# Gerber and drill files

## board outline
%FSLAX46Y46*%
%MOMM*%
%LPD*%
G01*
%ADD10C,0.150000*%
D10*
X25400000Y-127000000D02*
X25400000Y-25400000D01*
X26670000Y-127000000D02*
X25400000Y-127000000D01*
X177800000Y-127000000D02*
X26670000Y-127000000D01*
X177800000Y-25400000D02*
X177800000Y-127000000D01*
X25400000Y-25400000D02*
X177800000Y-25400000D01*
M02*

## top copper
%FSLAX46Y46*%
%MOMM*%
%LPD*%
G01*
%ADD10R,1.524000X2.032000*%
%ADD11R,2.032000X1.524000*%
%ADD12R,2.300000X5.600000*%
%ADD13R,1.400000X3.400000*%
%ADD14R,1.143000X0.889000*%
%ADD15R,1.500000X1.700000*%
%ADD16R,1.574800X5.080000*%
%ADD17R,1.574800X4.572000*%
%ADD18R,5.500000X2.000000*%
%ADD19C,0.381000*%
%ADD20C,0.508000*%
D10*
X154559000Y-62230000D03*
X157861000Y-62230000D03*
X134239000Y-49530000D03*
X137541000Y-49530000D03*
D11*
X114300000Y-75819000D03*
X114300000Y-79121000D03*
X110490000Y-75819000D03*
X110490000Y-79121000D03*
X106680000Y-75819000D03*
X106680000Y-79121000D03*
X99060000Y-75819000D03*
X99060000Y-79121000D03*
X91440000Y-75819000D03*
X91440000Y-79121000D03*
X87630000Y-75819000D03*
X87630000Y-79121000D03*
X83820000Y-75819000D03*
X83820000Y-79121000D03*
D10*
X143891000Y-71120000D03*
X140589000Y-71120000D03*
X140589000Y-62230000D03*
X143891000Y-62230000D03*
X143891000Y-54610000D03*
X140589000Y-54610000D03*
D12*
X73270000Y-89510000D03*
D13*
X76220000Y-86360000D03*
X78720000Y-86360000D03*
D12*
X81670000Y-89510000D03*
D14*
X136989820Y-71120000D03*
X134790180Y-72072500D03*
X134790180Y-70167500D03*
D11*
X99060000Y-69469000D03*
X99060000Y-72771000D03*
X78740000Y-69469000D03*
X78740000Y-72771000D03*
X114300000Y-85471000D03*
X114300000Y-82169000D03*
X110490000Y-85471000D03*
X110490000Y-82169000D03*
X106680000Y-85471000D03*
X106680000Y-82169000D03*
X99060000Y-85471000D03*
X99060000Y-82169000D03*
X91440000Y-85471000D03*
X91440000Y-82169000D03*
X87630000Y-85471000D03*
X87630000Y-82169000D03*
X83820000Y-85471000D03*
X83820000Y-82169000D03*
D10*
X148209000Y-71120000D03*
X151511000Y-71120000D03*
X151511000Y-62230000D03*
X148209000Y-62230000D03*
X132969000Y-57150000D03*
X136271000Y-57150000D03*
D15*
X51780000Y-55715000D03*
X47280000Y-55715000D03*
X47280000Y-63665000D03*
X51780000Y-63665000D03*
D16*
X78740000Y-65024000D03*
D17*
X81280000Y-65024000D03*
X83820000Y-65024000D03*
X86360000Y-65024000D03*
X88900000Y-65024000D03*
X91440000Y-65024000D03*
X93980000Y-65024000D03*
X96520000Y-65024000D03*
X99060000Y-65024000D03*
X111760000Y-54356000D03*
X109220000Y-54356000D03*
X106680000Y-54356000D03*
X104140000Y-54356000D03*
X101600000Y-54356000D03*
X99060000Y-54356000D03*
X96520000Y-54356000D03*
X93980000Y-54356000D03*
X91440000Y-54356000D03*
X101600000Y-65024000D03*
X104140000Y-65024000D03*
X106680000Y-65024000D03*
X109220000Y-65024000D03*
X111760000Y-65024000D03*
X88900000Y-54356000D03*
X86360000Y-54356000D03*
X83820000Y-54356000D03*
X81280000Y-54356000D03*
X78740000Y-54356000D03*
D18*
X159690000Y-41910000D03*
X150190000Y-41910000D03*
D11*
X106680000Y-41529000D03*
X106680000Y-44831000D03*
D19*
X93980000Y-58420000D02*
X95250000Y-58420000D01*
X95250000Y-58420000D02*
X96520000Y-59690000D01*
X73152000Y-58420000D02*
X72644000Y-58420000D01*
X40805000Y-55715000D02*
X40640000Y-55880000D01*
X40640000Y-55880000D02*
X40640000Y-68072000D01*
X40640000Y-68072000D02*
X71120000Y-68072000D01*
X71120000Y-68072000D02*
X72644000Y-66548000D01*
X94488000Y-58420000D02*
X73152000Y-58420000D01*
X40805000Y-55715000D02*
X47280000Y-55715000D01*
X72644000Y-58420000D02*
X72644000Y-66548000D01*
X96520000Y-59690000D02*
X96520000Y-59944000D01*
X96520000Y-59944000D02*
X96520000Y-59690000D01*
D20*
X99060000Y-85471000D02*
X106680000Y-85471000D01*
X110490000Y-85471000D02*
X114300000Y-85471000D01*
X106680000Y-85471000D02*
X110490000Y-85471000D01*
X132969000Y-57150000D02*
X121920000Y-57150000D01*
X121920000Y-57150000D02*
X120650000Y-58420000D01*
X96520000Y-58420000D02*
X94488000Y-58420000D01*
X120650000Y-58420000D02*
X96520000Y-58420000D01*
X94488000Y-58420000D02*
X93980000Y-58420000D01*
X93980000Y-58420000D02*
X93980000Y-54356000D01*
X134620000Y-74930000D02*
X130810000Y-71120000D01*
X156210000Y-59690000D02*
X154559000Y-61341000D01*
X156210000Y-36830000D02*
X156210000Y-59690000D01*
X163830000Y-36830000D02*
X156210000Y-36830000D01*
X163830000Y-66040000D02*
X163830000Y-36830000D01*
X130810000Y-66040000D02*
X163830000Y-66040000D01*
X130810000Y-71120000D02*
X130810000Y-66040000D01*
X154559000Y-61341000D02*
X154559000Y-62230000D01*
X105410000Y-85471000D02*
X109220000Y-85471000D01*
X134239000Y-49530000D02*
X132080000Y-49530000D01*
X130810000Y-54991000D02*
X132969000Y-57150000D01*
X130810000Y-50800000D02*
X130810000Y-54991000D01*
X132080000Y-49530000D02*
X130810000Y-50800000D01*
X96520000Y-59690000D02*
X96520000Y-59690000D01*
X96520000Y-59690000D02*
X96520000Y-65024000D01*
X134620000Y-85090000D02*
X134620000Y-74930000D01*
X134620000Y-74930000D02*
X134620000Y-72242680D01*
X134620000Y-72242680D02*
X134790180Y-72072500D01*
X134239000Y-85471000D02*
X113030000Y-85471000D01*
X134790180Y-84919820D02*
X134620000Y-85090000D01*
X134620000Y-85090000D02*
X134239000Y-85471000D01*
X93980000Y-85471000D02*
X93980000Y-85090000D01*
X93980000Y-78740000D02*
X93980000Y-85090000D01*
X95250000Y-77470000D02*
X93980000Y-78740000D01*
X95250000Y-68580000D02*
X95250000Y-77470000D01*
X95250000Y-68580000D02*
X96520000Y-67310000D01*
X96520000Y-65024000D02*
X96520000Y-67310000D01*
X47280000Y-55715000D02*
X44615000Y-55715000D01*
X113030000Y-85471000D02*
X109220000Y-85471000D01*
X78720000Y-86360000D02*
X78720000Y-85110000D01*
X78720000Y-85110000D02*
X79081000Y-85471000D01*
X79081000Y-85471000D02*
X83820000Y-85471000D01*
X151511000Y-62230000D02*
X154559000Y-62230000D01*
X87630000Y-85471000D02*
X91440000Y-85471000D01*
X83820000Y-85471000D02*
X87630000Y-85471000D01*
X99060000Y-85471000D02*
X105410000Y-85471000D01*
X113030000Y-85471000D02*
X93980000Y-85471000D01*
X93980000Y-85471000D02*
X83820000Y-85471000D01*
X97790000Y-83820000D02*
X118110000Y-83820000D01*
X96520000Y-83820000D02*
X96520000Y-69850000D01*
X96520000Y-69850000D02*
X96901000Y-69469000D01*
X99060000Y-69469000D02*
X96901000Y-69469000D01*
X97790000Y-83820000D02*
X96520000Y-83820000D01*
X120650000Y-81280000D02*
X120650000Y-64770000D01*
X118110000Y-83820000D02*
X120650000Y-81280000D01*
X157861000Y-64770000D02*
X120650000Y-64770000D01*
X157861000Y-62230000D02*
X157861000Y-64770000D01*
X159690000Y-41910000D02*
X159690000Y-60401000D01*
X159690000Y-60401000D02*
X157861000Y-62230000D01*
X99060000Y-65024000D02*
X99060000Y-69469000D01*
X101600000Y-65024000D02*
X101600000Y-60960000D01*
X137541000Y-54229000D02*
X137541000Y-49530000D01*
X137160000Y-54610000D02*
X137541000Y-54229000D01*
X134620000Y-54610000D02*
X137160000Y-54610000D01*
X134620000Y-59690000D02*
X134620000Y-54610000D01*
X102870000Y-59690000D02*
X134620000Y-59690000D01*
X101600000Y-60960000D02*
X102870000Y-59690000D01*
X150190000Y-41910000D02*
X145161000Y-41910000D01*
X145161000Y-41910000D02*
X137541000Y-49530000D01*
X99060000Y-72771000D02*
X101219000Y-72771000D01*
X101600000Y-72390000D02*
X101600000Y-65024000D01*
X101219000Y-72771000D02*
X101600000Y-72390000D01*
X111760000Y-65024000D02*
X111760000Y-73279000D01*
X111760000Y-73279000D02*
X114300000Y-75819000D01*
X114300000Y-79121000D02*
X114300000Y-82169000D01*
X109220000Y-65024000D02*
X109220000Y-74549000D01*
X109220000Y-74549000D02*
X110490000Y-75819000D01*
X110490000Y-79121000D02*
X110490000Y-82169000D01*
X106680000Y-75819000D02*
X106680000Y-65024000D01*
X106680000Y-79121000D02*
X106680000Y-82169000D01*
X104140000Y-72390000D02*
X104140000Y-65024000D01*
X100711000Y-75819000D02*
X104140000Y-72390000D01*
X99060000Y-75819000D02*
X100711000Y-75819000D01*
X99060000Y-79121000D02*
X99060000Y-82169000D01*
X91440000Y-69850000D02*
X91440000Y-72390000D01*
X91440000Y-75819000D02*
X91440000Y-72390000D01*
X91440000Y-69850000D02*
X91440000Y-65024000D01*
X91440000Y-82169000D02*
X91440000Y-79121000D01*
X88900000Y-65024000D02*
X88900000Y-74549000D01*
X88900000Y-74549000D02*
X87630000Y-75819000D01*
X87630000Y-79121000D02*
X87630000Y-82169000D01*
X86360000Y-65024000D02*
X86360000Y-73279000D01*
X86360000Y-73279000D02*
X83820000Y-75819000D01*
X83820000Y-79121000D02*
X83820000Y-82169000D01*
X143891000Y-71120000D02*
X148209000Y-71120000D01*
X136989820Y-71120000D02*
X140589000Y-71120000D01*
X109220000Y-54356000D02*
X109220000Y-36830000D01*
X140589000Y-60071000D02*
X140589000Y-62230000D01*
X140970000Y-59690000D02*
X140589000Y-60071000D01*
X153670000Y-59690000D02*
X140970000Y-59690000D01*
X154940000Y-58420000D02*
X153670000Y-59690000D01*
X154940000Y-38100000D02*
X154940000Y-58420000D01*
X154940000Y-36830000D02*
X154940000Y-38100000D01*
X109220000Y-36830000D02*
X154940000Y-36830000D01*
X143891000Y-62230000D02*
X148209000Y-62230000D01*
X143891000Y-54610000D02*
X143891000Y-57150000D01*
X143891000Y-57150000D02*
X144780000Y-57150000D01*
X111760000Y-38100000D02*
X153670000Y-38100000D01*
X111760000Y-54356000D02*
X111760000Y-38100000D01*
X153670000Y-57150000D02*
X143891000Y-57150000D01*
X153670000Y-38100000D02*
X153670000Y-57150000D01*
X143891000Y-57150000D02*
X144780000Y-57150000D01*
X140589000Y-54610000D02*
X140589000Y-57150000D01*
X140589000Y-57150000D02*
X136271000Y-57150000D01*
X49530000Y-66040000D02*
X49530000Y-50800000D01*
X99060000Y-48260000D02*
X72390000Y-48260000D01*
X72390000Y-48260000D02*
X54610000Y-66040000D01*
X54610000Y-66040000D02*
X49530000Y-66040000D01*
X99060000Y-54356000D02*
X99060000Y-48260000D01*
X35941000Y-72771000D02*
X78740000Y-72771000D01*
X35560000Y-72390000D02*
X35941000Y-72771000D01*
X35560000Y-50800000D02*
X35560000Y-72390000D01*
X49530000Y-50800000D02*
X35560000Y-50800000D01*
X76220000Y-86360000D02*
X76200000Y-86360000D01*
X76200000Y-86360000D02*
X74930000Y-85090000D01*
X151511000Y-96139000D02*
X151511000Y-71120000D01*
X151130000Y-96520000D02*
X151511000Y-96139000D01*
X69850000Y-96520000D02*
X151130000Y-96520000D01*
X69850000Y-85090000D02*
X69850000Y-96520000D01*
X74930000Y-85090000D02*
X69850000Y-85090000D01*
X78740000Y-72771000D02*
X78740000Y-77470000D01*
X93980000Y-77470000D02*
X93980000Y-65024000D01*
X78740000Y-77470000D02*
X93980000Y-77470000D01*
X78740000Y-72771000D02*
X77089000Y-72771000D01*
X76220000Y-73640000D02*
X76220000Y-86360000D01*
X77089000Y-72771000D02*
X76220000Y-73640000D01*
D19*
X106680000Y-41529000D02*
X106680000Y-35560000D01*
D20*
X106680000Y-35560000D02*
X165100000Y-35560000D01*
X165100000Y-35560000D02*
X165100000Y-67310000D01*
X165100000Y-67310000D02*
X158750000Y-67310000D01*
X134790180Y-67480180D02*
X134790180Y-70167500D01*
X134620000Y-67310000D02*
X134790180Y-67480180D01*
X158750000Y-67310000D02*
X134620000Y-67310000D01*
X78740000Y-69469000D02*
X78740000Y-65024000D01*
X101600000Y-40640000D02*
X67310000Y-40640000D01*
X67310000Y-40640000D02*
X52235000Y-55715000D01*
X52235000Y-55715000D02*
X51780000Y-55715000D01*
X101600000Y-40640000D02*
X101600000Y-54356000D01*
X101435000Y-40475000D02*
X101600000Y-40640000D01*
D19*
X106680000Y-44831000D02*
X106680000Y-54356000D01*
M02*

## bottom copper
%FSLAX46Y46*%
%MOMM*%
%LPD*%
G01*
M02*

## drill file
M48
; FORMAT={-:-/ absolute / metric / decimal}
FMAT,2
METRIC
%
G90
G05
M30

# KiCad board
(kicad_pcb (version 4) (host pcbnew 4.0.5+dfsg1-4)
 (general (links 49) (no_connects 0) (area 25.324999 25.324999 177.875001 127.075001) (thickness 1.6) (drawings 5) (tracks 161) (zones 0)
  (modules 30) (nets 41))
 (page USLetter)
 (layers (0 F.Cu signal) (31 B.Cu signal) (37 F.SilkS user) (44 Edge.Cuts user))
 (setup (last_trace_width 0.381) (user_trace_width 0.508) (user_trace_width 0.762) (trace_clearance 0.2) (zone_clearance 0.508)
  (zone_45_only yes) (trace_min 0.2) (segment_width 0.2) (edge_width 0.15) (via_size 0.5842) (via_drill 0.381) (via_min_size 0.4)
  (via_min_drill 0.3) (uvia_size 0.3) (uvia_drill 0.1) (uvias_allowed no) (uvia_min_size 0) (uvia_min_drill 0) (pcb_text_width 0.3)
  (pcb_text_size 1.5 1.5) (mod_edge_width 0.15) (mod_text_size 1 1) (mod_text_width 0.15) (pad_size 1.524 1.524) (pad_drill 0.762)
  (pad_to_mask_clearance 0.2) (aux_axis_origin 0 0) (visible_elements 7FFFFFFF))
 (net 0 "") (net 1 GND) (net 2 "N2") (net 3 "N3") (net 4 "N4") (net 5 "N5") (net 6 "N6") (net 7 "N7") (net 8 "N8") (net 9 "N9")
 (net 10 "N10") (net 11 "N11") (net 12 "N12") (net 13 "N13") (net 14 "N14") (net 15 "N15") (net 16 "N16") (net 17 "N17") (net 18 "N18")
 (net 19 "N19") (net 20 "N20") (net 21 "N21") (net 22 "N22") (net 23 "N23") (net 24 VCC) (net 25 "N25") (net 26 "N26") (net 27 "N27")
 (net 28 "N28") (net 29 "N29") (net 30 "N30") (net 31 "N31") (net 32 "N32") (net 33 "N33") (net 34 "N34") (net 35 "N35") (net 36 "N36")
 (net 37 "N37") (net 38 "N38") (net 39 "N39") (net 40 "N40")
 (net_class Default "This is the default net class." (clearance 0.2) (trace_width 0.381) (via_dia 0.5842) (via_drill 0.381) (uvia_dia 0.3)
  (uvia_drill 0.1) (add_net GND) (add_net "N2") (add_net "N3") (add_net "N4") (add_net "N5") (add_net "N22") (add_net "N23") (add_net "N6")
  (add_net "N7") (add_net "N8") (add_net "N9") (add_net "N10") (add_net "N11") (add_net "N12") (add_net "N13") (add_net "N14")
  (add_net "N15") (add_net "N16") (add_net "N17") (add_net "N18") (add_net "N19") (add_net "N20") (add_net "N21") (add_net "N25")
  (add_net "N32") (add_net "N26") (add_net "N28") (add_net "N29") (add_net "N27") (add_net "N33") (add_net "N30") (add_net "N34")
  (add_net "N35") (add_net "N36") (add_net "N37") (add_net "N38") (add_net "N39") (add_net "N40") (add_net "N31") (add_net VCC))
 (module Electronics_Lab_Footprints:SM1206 (layer F.Cu) (at 156.21 62.23)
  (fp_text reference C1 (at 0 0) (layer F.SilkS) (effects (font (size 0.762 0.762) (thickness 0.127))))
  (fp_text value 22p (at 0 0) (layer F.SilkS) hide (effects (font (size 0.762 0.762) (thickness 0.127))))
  (pad 1 smd rect (at -1.651 0) (size 1.524 2.032) (layers F.Cu) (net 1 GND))
  (pad 2 smd rect (at 1.651 0) (size 1.524 2.032) (layers F.Cu) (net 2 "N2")))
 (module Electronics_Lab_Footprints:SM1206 (layer F.Cu) (at 135.89 49.53)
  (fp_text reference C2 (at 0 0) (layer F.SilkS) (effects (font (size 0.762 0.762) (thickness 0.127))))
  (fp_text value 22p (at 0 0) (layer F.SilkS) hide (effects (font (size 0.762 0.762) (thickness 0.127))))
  (pad 1 smd rect (at -1.651 0) (size 1.524 2.032) (layers F.Cu) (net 1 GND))
  (pad 2 smd rect (at 1.651 0) (size 1.524 2.032) (layers F.Cu) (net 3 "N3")))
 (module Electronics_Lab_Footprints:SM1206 (layer F.Cu) (at 114.3 77.47 270)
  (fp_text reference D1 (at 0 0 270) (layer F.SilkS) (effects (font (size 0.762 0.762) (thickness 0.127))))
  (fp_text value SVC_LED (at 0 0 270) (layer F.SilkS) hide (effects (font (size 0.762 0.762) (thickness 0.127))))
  (pad 1 smd rect (at -1.651 0 270) (size 1.524 2.032) (layers F.Cu) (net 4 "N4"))
  (pad 2 smd rect (at 1.651 0 270) (size 1.524 2.032) (layers F.Cu) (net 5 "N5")))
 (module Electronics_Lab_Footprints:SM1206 (layer F.Cu) (at 110.49 77.47 270)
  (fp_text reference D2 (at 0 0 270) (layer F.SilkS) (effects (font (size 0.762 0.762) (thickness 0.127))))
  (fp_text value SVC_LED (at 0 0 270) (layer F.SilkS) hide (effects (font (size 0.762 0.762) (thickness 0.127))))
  (pad 1 smd rect (at -1.651 0 270) (size 1.524 2.032) (layers F.Cu) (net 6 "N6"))
  (pad 2 smd rect (at 1.651 0 270) (size 1.524 2.032) (layers F.Cu) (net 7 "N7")))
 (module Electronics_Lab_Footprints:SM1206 (layer F.Cu) (at 106.68 77.47 270)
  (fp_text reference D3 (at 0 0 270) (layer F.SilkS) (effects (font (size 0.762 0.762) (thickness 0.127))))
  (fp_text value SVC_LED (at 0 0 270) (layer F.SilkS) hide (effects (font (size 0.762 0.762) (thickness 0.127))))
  (pad 1 smd rect (at -1.651 0 270) (size 1.524 2.032) (layers F.Cu) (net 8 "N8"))
  (pad 2 smd rect (at 1.651 0 270) (size 1.524 2.032) (layers F.Cu) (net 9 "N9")))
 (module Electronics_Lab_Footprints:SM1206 (layer F.Cu) (at 99.06 77.47 270)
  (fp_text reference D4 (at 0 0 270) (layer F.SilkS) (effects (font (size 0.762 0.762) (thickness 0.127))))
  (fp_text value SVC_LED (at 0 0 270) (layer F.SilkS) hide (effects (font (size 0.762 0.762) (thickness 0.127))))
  (pad 1 smd rect (at -1.651 0 270) (size 1.524 2.032) (layers F.Cu) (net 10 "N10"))
  (pad 2 smd rect (at 1.651 0 270) (size 1.524 2.032) (layers F.Cu) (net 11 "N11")))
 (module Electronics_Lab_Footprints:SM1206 (layer F.Cu) (at 91.44 77.47 270)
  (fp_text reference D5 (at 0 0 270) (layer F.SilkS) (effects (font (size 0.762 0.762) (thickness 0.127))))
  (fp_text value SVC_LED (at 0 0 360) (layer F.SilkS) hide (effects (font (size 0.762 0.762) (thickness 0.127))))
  (pad 1 smd rect (at -1.651 0 270) (size 1.524 2.032) (layers F.Cu) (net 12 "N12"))
  (pad 2 smd rect (at 1.651 0 270) (size 1.524 2.032) (layers F.Cu) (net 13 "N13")))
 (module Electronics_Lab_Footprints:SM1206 (layer F.Cu) (at 87.63 77.47 270)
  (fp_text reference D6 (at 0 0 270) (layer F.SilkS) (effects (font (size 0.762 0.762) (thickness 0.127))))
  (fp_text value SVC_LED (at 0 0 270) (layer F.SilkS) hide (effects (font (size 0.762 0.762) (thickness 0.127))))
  (pad 1 smd rect (at -1.651 0 270) (size 1.524 2.032) (layers F.Cu) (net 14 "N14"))
  (pad 2 smd rect (at 1.651 0 270) (size 1.524 2.032) (layers F.Cu) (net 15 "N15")))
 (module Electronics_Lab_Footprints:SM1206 (layer F.Cu) (at 83.82 77.47 270)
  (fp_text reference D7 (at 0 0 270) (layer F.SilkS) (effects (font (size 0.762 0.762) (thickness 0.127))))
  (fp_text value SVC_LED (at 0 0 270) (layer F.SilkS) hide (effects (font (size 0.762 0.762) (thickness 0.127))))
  (pad 1 smd rect (at -1.651 0 270) (size 1.524 2.032) (layers F.Cu) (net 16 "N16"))
  (pad 2 smd rect (at 1.651 0 270) (size 1.524 2.032) (layers F.Cu) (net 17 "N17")))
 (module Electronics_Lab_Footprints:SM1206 (layer F.Cu) (at 142.24 71.12 180)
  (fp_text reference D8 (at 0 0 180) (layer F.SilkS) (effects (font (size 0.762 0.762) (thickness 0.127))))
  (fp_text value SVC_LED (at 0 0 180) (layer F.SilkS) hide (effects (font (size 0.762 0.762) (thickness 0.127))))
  (pad 1 smd rect (at -1.651 0 180) (size 1.524 2.032) (layers F.Cu) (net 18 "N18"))
  (pad 2 smd rect (at 1.651 0 180) (size 1.524 2.032) (layers F.Cu) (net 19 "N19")))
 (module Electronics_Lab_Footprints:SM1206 (layer F.Cu) (at 142.24 62.23)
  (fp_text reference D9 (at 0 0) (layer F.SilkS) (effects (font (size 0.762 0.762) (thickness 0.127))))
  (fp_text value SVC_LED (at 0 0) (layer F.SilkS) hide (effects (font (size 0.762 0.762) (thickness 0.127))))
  (pad 1 smd rect (at -1.651 0) (size 1.524 2.032) (layers F.Cu) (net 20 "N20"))
  (pad 2 smd rect (at 1.651 0) (size 1.524 2.032) (layers F.Cu) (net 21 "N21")))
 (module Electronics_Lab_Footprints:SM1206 (layer F.Cu) (at 142.24 54.61 180)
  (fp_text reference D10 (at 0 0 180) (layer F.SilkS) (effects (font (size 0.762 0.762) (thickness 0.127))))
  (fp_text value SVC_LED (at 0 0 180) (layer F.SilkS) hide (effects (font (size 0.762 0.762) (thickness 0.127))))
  (pad 1 smd rect (at -1.651 0 180) (size 1.524 2.032) (layers F.Cu) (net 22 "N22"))
  (pad 2 smd rect (at 1.651 0 180) (size 1.524 2.032) (layers F.Cu) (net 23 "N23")))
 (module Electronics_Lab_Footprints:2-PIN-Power (layer F.Cu) (at 77.47 86.36)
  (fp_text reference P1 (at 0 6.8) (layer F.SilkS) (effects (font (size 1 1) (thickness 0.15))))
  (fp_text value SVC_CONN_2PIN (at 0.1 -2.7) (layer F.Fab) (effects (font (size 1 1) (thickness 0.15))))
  (pad "" smd rect (at -4.2 3.15) (size 2.3 5.6) (layers F.Cu))
  (pad 1 smd rect (at -1.25 0) (size 1.4 3.4) (layers F.Cu) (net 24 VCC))
  (pad 2 smd rect (at 1.25 0) (size 1.4 3.4) (layers F.Cu) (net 1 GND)) (pad "" smd rect (at 4.2 3.15) (size 2.3 5.6) (layers F.Cu)))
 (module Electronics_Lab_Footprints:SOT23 (layer F.Cu) (at 135.89 71.12 270)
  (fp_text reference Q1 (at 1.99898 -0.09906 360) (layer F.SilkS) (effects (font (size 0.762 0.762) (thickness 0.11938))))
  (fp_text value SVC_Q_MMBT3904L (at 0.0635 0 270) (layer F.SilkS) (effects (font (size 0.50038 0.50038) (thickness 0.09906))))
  (pad 3 smd rect (at 0 -1.09982 270) (size 0.889 1.143) (layers F.Cu) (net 19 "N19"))
  (pad 2 smd rect (at 0.9525 1.09982 270) (size 0.889 1.143) (layers F.Cu) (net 1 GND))
  (pad 1 smd rect (at -0.9525 1.09982 270) (size 0.889 1.143) (layers F.Cu) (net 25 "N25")))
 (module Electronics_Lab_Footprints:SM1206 (layer F.Cu) (at 99.06 71.12 270)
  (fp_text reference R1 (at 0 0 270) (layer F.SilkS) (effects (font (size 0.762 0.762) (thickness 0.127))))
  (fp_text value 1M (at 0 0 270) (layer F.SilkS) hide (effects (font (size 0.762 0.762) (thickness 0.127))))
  (pad 1 smd rect (at -1.651 0 270) (size 1.524 2.032) (layers F.Cu) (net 2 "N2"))
  (pad 2 smd rect (at 1.651 0 270) (size 1.524 2.032) (layers F.Cu) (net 3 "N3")))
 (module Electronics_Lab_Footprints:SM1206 (layer F.Cu) (at 78.74 71.12 270)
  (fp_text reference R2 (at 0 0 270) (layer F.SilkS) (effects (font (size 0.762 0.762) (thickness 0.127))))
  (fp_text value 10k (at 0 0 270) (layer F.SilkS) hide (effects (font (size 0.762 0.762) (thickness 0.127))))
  (pad 1 smd rect (at -1.651 0 270) (size 1.524 2.032) (layers F.Cu) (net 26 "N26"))
  (pad 2 smd rect (at 1.651 0 270) (size 1.524 2.032) (layers F.Cu) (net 24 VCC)))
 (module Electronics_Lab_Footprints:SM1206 (layer F.Cu) (at 114.3 83.82 90)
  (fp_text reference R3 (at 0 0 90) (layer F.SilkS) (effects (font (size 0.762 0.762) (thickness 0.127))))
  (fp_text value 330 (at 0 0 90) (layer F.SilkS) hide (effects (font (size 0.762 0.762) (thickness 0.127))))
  (pad 1 smd rect (at -1.651 0 90) (size 1.524 2.032) (layers F.Cu) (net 1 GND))
  (pad 2 smd rect (at 1.651 0 90) (size 1.524 2.032) (layers F.Cu) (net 5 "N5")))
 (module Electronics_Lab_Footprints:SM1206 (layer F.Cu) (at 110.49 83.82 90)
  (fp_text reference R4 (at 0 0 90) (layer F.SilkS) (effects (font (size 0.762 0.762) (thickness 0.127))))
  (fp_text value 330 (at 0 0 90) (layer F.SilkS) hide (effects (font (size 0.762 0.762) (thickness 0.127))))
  (pad 1 smd rect (at -1.651 0 90) (size 1.524 2.032) (layers F.Cu) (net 1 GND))
  (pad 2 smd rect (at 1.651 0 90) (size 1.524 2.032) (layers F.Cu) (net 7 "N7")))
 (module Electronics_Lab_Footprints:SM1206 (layer F.Cu) (at 106.68 83.82 90)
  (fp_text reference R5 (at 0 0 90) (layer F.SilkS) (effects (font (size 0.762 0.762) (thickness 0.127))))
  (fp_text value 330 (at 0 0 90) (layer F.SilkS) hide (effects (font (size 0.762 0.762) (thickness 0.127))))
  (pad 1 smd rect (at -1.651 0 90) (size 1.524 2.032) (layers F.Cu) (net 1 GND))
  (pad 2 smd rect (at 1.651 0 90) (size 1.524 2.032) (layers F.Cu) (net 9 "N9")))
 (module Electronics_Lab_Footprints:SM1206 (layer F.Cu) (at 99.06 83.82 90)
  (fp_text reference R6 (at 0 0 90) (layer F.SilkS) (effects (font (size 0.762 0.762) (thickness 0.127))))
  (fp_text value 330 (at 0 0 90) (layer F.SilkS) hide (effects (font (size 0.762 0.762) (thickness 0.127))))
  (pad 1 smd rect (at -1.651 0 90) (size 1.524 2.032) (layers F.Cu) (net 1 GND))
  (pad 2 smd rect (at 1.651 0 90) (size 1.524 2.032) (layers F.Cu) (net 11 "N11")))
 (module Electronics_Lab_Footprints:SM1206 (layer F.Cu) (at 91.44 83.82 90)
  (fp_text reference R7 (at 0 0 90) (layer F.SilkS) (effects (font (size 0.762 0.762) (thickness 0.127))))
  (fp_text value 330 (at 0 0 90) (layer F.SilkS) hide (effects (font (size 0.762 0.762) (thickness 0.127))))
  (pad 1 smd rect (at -1.651 0 90) (size 1.524 2.032) (layers F.Cu) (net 1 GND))
  (pad 2 smd rect (at 1.651 0 90) (size 1.524 2.032) (layers F.Cu) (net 13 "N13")))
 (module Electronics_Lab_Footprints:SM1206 (layer F.Cu) (at 87.63 83.82 90)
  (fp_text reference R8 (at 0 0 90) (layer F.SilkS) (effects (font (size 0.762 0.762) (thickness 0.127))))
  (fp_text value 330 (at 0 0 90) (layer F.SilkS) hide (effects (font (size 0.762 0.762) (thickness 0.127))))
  (pad 1 smd rect (at -1.651 0 90) (size 1.524 2.032) (layers F.Cu) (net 1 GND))
  (pad 2 smd rect (at 1.651 0 90) (size 1.524 2.032) (layers F.Cu) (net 15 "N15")))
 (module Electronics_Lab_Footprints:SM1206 (layer F.Cu) (at 83.82 83.82 90)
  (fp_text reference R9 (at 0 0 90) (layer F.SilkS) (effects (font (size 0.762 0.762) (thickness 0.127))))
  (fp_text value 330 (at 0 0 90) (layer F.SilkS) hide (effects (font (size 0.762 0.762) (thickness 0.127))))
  (pad 1 smd rect (at -1.651 0 90) (size 1.524 2.032) (layers F.Cu) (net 1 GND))
  (pad 2 smd rect (at 1.651 0 90) (size 1.524 2.032) (layers F.Cu) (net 17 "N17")))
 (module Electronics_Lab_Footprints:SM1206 (layer F.Cu) (at 149.86 71.12)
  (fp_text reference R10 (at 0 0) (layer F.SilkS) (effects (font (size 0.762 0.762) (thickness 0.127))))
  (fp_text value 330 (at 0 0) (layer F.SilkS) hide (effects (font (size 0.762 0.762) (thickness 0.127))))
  (pad 1 smd rect (at -1.651 0) (size 1.524 2.032) (layers F.Cu) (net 18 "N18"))
  (pad 2 smd rect (at 1.651 0) (size 1.524 2.032) (layers F.Cu) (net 24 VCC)))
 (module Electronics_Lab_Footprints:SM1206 (layer F.Cu) (at 149.86 62.23 180)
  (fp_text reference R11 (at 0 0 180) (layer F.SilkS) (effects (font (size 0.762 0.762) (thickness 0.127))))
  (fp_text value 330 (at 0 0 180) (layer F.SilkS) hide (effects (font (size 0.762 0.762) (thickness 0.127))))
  (pad 1 smd rect (at -1.651 0 180) (size 1.524 2.032) (layers F.Cu) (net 1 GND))
  (pad 2 smd rect (at 1.651 0 180) (size 1.524 2.032) (layers F.Cu) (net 21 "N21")))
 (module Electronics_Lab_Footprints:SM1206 (layer F.Cu) (at 134.62 57.15)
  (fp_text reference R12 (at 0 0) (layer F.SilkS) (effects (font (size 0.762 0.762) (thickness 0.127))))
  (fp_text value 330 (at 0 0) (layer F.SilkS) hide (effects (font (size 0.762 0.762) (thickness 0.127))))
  (pad 1 smd rect (at -1.651 0) (size 1.524 2.032) (layers F.Cu) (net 1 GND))
  (pad 2 smd rect (at 1.651 0) (size 1.524 2.032) (layers F.Cu) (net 23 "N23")))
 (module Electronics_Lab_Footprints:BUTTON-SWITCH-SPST (layer F.Cu) (at 49.53 59.69 90)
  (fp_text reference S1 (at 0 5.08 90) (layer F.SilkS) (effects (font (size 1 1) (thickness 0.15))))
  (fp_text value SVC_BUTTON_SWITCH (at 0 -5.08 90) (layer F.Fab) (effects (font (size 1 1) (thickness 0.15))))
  (pad 4 smd rect (at 3.975 2.25 90) (size 1.7 1.5) (layers F.Cu) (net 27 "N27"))
  (pad 2 smd rect (at 3.975 -2.25 90) (size 1.7 1.5) (layers F.Cu) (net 1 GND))
  (pad 1 smd rect (at -3.975 -2.25 90) (size 1.7 1.5) (layers F.Cu) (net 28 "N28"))
  (pad 3 smd rect (at -3.975 2.25 90) (size 1.7 1.5) (layers F.Cu) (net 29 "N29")))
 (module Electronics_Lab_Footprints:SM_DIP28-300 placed (layer F.Cu) (at 95.25 59.69)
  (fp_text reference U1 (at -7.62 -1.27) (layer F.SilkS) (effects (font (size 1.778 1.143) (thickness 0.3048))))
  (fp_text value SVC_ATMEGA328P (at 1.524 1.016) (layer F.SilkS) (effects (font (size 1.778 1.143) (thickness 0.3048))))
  (pad 1 smd rect (at -16.51 5.334) (size 1.5748 5.08) (layers F.Cu) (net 26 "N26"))
  (pad 2 smd rect (at -13.97 5.334) (size 1.5748 4.572) (layers F.Cu) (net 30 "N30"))
  (pad 3 smd rect (at -11.43 5.334) (size 1.5748 4.572) (layers F.Cu) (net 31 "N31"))
  (pad 4 smd rect (at -8.89 5.334) (size 1.5748 4.572) (layers F.Cu) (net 16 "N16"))
  (pad 5 smd rect (at -6.35 5.334) (size 1.5748 4.572) (layers F.Cu) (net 14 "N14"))
  (pad 6 smd rect (at -3.81 5.334) (size 1.5748 4.572) (layers F.Cu) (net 12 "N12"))
  (pad 7 smd rect (at -1.27 5.334) (size 1.5748 4.572) (layers F.Cu) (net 24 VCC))
  (pad 8 smd rect (at 1.27 5.334) (size 1.5748 4.572) (layers F.Cu) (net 1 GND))
  (pad 9 smd rect (at 3.81 5.334) (size 1.5748 4.572) (layers F.Cu) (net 2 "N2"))
  (pad 15 smd rect (at 16.51 -5.334) (size 1.5748 4.572) (layers F.Cu) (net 22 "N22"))
  (pad 16 smd rect (at 13.97 -5.334) (size 1.5748 4.572) (layers F.Cu) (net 20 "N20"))
  (pad 17 smd rect (at 11.43 -5.334) (size 1.5748 4.572) (layers F.Cu) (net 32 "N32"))
  (pad 18 smd rect (at 8.89 -5.334) (size 1.5748 4.572) (layers F.Cu) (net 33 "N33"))
  (pad 19 smd rect (at 6.35 -5.334) (size 1.5748 4.572) (layers F.Cu) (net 27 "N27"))
  (pad 20 smd rect (at 3.81 -5.334) (size 1.5748 4.572) (layers F.Cu) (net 24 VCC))
  (pad 21 smd rect (at 1.27 -5.334) (size 1.5748 4.572) (layers F.Cu) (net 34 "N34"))
  (pad 22 smd rect (at -1.27 -5.334) (size 1.5748 4.572) (layers F.Cu) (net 1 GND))
  (pad 23 smd rect (at -3.81 -5.334) (size 1.5748 4.572) (layers F.Cu) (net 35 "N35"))
  (pad 10 smd rect (at 6.35 5.334) (size 1.5748 4.572) (layers F.Cu) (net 3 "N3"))
  (pad 11 smd rect (at 8.89 5.334) (size 1.5748 4.572) (layers F.Cu) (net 10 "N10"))
  (pad 12 smd rect (at 11.43 5.334) (size 1.5748 4.572) (layers F.Cu) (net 8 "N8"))
  (pad 13 smd rect (at 13.97 5.334) (size 1.5748 4.572) (layers F.Cu) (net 6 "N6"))
  (pad 14 smd rect (at 16.51 5.334) (size 1.5748 4.572) (layers F.Cu) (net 4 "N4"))
  (pad 24 smd rect (at -6.35 -5.334) (size 1.5748 4.572) (layers F.Cu) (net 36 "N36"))
  (pad 25 smd rect (at -8.89 -5.334) (size 1.5748 4.572) (layers F.Cu) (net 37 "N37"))
  (pad 26 smd rect (at -11.43 -5.334) (size 1.5748 4.572) (layers F.Cu) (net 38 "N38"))
  (pad 27 smd rect (at -13.97 -5.334) (size 1.5748 4.572) (layers F.Cu) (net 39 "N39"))
  (pad 28 smd rect (at -16.51 -5.334) (size 1.5748 4.572) (layers F.Cu) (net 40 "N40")))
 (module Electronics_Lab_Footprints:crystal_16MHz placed (layer F.Cu) (at 154.94 41.91 180)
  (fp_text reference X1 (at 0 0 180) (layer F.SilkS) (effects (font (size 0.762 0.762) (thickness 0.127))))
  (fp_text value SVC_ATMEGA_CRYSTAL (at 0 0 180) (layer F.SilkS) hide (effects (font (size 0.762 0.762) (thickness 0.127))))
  (pad 1 smd rect (at -4.75 0 180) (size 5.5 2) (layers F.Cu) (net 2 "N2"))
  (pad 2 smd rect (at 4.75 0 180) (size 5.5 2) (layers F.Cu) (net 3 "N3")))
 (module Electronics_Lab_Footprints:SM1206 (layer F.Cu) (at 106.68 43.18 270)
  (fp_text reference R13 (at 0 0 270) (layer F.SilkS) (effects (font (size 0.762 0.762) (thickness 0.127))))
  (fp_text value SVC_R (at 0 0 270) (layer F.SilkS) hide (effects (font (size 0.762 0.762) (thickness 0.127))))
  (pad 1 smd rect (at -1.651 0 270) (size 1.524 2.032) (layers F.Cu) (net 25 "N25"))
  (pad 2 smd rect (at 1.651 0 270) (size 1.524 2.032) (layers F.Cu) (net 32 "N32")))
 (gr_line (start 25.4 127) (end 25.4 25.4) (angle 90) (layer Edge.Cuts) (width 0.15))
 (gr_line (start 26.67 127) (end 25.4 127) (angle 90) (layer Edge.Cuts) (width 0.15))
 (gr_line (start 177.8 127) (end 26.67 127) (angle 90) (layer Edge.Cuts) (width 0.15))
 (gr_line (start 177.8 25.4) (end 177.8 127) (angle 90) (layer Edge.Cuts) (width 0.15))
 (gr_line (start 25.4 25.4) (end 177.8 25.4) (angle 90) (layer Edge.Cuts) (width 0.15))
 (segment (start 93.98 58.42) (end 95.25 58.42) (width 0.381) (layer F.Cu) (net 1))
 (segment (start 95.25 58.42) (end 96.52 59.69) (width 0.381) (layer F.Cu) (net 1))
 (segment (start 73.152 58.42) (end 72.644 58.42) (width 0.381) (layer F.Cu) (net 1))
 (segment (start 40.805 55.715) (end 40.64 55.88) (width 0.381) (layer F.Cu) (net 1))
 (segment (start 40.64 55.88) (end 40.64 68.072) (width 0.381) (layer F.Cu) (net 1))
 (segment (start 40.64 68.072) (end 71.12 68.072) (width 0.381) (layer F.Cu) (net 1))
 (segment (start 71.12 68.072) (end 72.644 66.548) (width 0.381) (layer F.Cu) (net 1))
 (segment (start 94.488 58.42) (end 73.152 58.42) (width 0.381) (layer F.Cu) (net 1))
 (segment (start 40.805 55.715) (end 47.28 55.715) (width 0.381) (layer F.Cu) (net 1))
 (segment (start 72.644 58.42) (end 72.644 66.548) (width 0.381) (layer F.Cu) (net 1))
 (segment (start 96.52 59.69) (end 96.52 59.944) (width 0.381) (layer F.Cu) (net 1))
 (segment (start 96.52 59.944) (end 96.52 59.69) (width 0.381) (layer F.Cu) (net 1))
 (segment (start 99.06 85.471) (end 106.68 85.471) (width 0.508) (layer F.Cu) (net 1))
 (segment (start 110.49 85.471) (end 114.3 85.471) (width 0.508) (layer F.Cu) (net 1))
 (segment (start 106.68 85.471) (end 110.49 85.471) (width 0.508) (layer F.Cu) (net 1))
 (segment (start 132.969 57.15) (end 121.92 57.15) (width 0.508) (layer F.Cu) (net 1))
 (segment (start 121.92 57.15) (end 120.65 58.42) (width 0.508) (layer F.Cu) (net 1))
 (segment (start 96.52 58.42) (end 94.488 58.42) (width 0.508) (layer F.Cu) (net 1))
 (segment (start 120.65 58.42) (end 96.52 58.42) (width 0.508) (layer F.Cu) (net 1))
 (segment (start 94.488 58.42) (end 93.98 58.42) (width 0.508) (layer F.Cu) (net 1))
 (segment (start 93.98 58.42) (end 93.98 54.356) (width 0.508) (layer F.Cu) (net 1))
 (segment (start 134.62 74.93) (end 130.81 71.12) (width 0.508) (layer F.Cu) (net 1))
 (segment (start 156.21 59.69) (end 154.559 61.341) (width 0.508) (layer F.Cu) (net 1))
 (segment (start 156.21 36.83) (end 156.21 59.69) (width 0.508) (layer F.Cu) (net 1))
 (segment (start 163.83 36.83) (end 156.21 36.83) (width 0.508) (layer F.Cu) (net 1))
 (segment (start 163.83 66.04) (end 163.83 36.83) (width 0.508) (layer F.Cu) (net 1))
 (segment (start 130.81 66.04) (end 163.83 66.04) (width 0.508) (layer F.Cu) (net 1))
 (segment (start 130.81 71.12) (end 130.81 66.04) (width 0.508) (layer F.Cu) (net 1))
 (segment (start 154.559 61.341) (end 154.559 62.23) (width 0.508) (layer F.Cu) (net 1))
 (segment (start 105.41 85.471) (end 109.22 85.471) (width 0.508) (layer F.Cu) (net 1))
 (segment (start 134.239 49.53) (end 132.08 49.53) (width 0.508) (layer F.Cu) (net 1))
 (segment (start 130.81 54.991) (end 132.969 57.15) (width 0.508) (layer F.Cu) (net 1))
 (segment (start 130.81 50.8) (end 130.81 54.991) (width 0.508) (layer F.Cu) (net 1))
 (segment (start 132.08 49.53) (end 130.81 50.8) (width 0.508) (layer F.Cu) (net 1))
 (segment (start 96.52 59.69) (end 96.52 59.69) (width 0.508) (layer F.Cu) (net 1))
 (segment (start 96.52 59.69) (end 96.52 65.024) (width 0.508) (layer F.Cu) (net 1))
 (segment (start 134.62 85.09) (end 134.62 74.93) (width 0.508) (layer F.Cu) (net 1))
 (segment (start 134.62 74.93) (end 134.62 72.24268) (width 0.508) (layer F.Cu) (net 1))
 (segment (start 134.62 72.24268) (end 134.79018 72.0725) (width 0.508) (layer F.Cu) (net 1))
 (segment (start 134.239 85.471) (end 113.03 85.471) (width 0.508) (layer F.Cu) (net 1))
 (segment (start 134.79018 84.91982) (end 134.62 85.09) (width 0.508) (layer F.Cu) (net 1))
 (segment (start 134.62 85.09) (end 134.239 85.471) (width 0.508) (layer F.Cu) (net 1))
 (segment (start 93.98 85.471) (end 93.98 85.09) (width 0.508) (layer F.Cu) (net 1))
 (segment (start 93.98 78.74) (end 93.98 85.09) (width 0.508) (layer F.Cu) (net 1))
 (segment (start 95.25 77.47) (end 93.98 78.74) (width 0.508) (layer F.Cu) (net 1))
 (segment (start 95.25 68.58) (end 95.25 77.47) (width 0.508) (layer F.Cu) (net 1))
 (segment (start 95.25 68.58) (end 96.52 67.31) (width 0.508) (layer F.Cu) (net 1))
 (segment (start 96.52 65.024) (end 96.52 67.31) (width 0.508) (layer F.Cu) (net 1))
 (segment (start 47.28 55.715) (end 44.615 55.715) (width 0.508) (layer F.Cu) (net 1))
 (segment (start 113.03 85.471) (end 109.22 85.471) (width 0.508) (layer F.Cu) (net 1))
 (segment (start 78.72 86.36) (end 78.72 85.11) (width 0.508) (layer F.Cu) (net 1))
 (segment (start 78.72 85.11) (end 79.081 85.471) (width 0.508) (layer F.Cu) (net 1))
 (segment (start 79.081 85.471) (end 83.82 85.471) (width 0.508) (layer F.Cu) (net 1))
 (segment (start 151.511 62.23) (end 154.559 62.23) (width 0.508) (layer F.Cu) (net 1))
 (segment (start 87.63 85.471) (end 91.44 85.471) (width 0.508) (layer F.Cu) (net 1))
 (segment (start 83.82 85.471) (end 87.63 85.471) (width 0.508) (layer F.Cu) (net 1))
 (segment (start 99.06 85.471) (end 105.41 85.471) (width 0.508) (layer F.Cu) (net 1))
 (segment (start 113.03 85.471) (end 93.98 85.471) (width 0.508) (layer F.Cu) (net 1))
 (segment (start 93.98 85.471) (end 83.82 85.471) (width 0.508) (layer F.Cu) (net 1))
 (segment (start 97.79 83.82) (end 118.11 83.82) (width 0.508) (layer F.Cu) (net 2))
 (segment (start 96.52 83.82) (end 96.52 69.85) (width 0.508) (layer F.Cu) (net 2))
 (segment (start 96.52 69.85) (end 96.901 69.469) (width 0.508) (layer F.Cu) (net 2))
 (segment (start 99.06 69.469) (end 96.901 69.469) (width 0.508) (layer F.Cu) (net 2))
 (segment (start 97.79 83.82) (end 96.52 83.82) (width 0.508) (layer F.Cu) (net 2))
 (segment (start 120.65 81.28) (end 120.65 64.77) (width 0.508) (layer F.Cu) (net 2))
 (segment (start 118.11 83.82) (end 120.65 81.28) (width 0.508) (layer F.Cu) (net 2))
 (segment (start 157.861 64.77) (end 120.65 64.77) (width 0.508) (layer F.Cu) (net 2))
 (segment (start 157.861 62.23) (end 157.861 64.77) (width 0.508) (layer F.Cu) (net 2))
 (segment (start 159.69 41.91) (end 159.69 60.401) (width 0.508) (layer F.Cu) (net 2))
 (segment (start 159.69 60.401) (end 157.861 62.23) (width 0.508) (layer F.Cu) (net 2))
 (segment (start 99.06 65.024) (end 99.06 69.469) (width 0.508) (layer F.Cu) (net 2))
 (segment (start 101.6 65.024) (end 101.6 60.96) (width 0.508) (layer F.Cu) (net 3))
 (segment (start 137.541 54.229) (end 137.541 49.53) (width 0.508) (layer F.Cu) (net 3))
 (segment (start 137.16 54.61) (end 137.541 54.229) (width 0.508) (layer F.Cu) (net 3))
 (segment (start 134.62 54.61) (end 137.16 54.61) (width 0.508) (layer F.Cu) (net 3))
 (segment (start 134.62 59.69) (end 134.62 54.61) (width 0.508) (layer F.Cu) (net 3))
 (segment (start 102.87 59.69) (end 134.62 59.69) (width 0.508) (layer F.Cu) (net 3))
 (segment (start 101.6 60.96) (end 102.87 59.69) (width 0.508) (layer F.Cu) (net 3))
 (segment (start 150.19 41.91) (end 145.161 41.91) (width 0.508) (layer F.Cu) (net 3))
 (segment (start 145.161 41.91) (end 137.541 49.53) (width 0.508) (layer F.Cu) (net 3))
 (segment (start 99.06 72.771) (end 101.219 72.771) (width 0.508) (layer F.Cu) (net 3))
 (segment (start 101.6 72.39) (end 101.6 65.024) (width 0.508) (layer F.Cu) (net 3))
 (segment (start 101.219 72.771) (end 101.6 72.39) (width 0.508) (layer F.Cu) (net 3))
 (segment (start 111.76 65.024) (end 111.76 73.279) (width 0.508) (layer F.Cu) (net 4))
 (segment (start 111.76 73.279) (end 114.3 75.819) (width 0.508) (layer F.Cu) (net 4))
 (segment (start 114.3 79.121) (end 114.3 82.169) (width 0.508) (layer F.Cu) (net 5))
 (segment (start 109.22 65.024) (end 109.22 74.549) (width 0.508) (layer F.Cu) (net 6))
 (segment (start 109.22 74.549) (end 110.49 75.819) (width 0.508) (layer F.Cu) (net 6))
 (segment (start 110.49 79.121) (end 110.49 82.169) (width 0.508) (layer F.Cu) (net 7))
 (segment (start 106.68 75.819) (end 106.68 65.024) (width 0.508) (layer F.Cu) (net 8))
 (segment (start 106.68 79.121) (end 106.68 82.169) (width 0.508) (layer F.Cu) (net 9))
 (segment (start 104.14 72.39) (end 104.14 65.024) (width 0.508) (layer F.Cu) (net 10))
 (segment (start 100.711 75.819) (end 104.14 72.39) (width 0.508) (layer F.Cu) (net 10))
 (segment (start 99.06 75.819) (end 100.711 75.819) (width 0.508) (layer F.Cu) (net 10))
 (segment (start 99.06 79.121) (end 99.06 82.169) (width 0.508) (layer F.Cu) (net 11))
 (segment (start 91.44 69.85) (end 91.44 72.39) (width 0.508) (layer F.Cu) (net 12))
 (segment (start 91.44 75.819) (end 91.44 72.39) (width 0.508) (layer F.Cu) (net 12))
 (segment (start 91.44 69.85) (end 91.44 65.024) (width 0.508) (layer F.Cu) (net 12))
 (segment (start 91.44 82.169) (end 91.44 79.121) (width 0.508) (layer F.Cu) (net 13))
 (segment (start 88.9 65.024) (end 88.9 74.549) (width 0.508) (layer F.Cu) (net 14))
 (segment (start 88.9 74.549) (end 87.63 75.819) (width 0.508) (layer F.Cu) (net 14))
 (segment (start 87.63 79.121) (end 87.63 82.169) (width 0.508) (layer F.Cu) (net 15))
 (segment (start 86.36 65.024) (end 86.36 73.279) (width 0.508) (layer F.Cu) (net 16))
 (segment (start 86.36 73.279) (end 83.82 75.819) (width 0.508) (layer F.Cu) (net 16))
 (segment (start 83.82 79.121) (end 83.82 82.169) (width 0.508) (layer F.Cu) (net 17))
 (segment (start 143.891 71.12) (end 148.209 71.12) (width 0.508) (layer F.Cu) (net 18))
 (segment (start 136.98982 71.12) (end 140.589 71.12) (width 0.508) (layer F.Cu) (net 19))
 (segment (start 109.22 54.356) (end 109.22 36.83) (width 0.508) (layer F.Cu) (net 20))
 (segment (start 140.589 60.071) (end 140.589 62.23) (width 0.508) (layer F.Cu) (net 20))
 (segment (start 140.97 59.69) (end 140.589 60.071) (width 0.508) (layer F.Cu) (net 20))
 (segment (start 153.67 59.69) (end 140.97 59.69) (width 0.508) (layer F.Cu) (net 20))
 (segment (start 154.94 58.42) (end 153.67 59.69) (width 0.508) (layer F.Cu) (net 20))
 (segment (start 154.94 38.1) (end 154.94 58.42) (width 0.508) (layer F.Cu) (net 20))
 (segment (start 154.94 36.83) (end 154.94 38.1) (width 0.508) (layer F.Cu) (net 20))
 (segment (start 109.22 36.83) (end 154.94 36.83) (width 0.508) (layer F.Cu) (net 20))
 (segment (start 143.891 62.23) (end 148.209 62.23) (width 0.508) (layer F.Cu) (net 21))
 (segment (start 143.891 54.61) (end 143.891 57.15) (width 0.508) (layer F.Cu) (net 22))
 (segment (start 143.891 57.15) (end 144.78 57.15) (width 0.508) (layer F.Cu) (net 22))
 (segment (start 111.76 38.1) (end 153.67 38.1) (width 0.508) (layer F.Cu) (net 22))
 (segment (start 111.76 54.356) (end 111.76 38.1) (width 0.508) (layer F.Cu) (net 22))
 (segment (start 153.67 57.15) (end 143.891 57.15) (width 0.508) (layer F.Cu) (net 22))
 (segment (start 153.67 38.1) (end 153.67 57.15) (width 0.508) (layer F.Cu) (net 22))
 (segment (start 143.891 57.15) (end 144.78 57.15) (width 0.508) (layer F.Cu) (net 22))
 (segment (start 140.589 54.61) (end 140.589 57.15) (width 0.508) (layer F.Cu) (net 23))
 (segment (start 140.589 57.15) (end 136.271 57.15) (width 0.508) (layer F.Cu) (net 23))
 (segment (start 49.53 66.04) (end 49.53 50.8) (width 0.508) (layer F.Cu) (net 24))
 (segment (start 99.06 48.26) (end 72.39 48.26) (width 0.508) (layer F.Cu) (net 24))
 (segment (start 72.39 48.26) (end 54.61 66.04) (width 0.508) (layer F.Cu) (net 24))
 (segment (start 54.61 66.04) (end 49.53 66.04) (width 0.508) (layer F.Cu) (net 24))
 (segment (start 99.06 54.356) (end 99.06 48.26) (width 0.508) (layer F.Cu) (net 24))
 (segment (start 35.941 72.771) (end 78.74 72.771) (width 0.508) (layer F.Cu) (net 24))
 (segment (start 35.56 72.39) (end 35.941 72.771) (width 0.508) (layer F.Cu) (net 24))
 (segment (start 35.56 50.8) (end 35.56 72.39) (width 0.508) (layer F.Cu) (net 24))
 (segment (start 49.53 50.8) (end 35.56 50.8) (width 0.508) (layer F.Cu) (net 24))
 (segment (start 76.22 86.36) (end 76.2 86.36) (width 0.508) (layer F.Cu) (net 24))
 (segment (start 76.2 86.36) (end 74.93 85.09) (width 0.508) (layer F.Cu) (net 24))
 (segment (start 151.511 96.139) (end 151.511 71.12) (width 0.508) (layer F.Cu) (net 24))
 (segment (start 151.13 96.52) (end 151.511 96.139) (width 0.508) (layer F.Cu) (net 24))
 (segment (start 69.85 96.52) (end 151.13 96.52) (width 0.508) (layer F.Cu) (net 24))
 (segment (start 69.85 85.09) (end 69.85 96.52) (width 0.508) (layer F.Cu) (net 24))
 (segment (start 74.93 85.09) (end 69.85 85.09) (width 0.508) (layer F.Cu) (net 24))
 (segment (start 78.74 72.771) (end 78.74 77.47) (width 0.508) (layer F.Cu) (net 24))
 (segment (start 93.98 77.47) (end 93.98 65.024) (width 0.508) (layer F.Cu) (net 24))
 (segment (start 78.74 77.47) (end 93.98 77.47) (width 0.508) (layer F.Cu) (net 24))
 (segment (start 78.74 72.771) (end 77.089 72.771) (width 0.508) (layer F.Cu) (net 24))
 (segment (start 76.22 73.64) (end 76.22 86.36) (width 0.508) (layer F.Cu) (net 24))
 (segment (start 77.089 72.771) (end 76.22 73.64) (width 0.508) (layer F.Cu) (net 24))
 (segment (start 106.68 41.529) (end 106.68 35.56) (width 0.381) (layer F.Cu) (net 25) (status 400000))
 (segment (start 106.68 35.56) (end 165.1 35.56) (width 0.508) (layer F.Cu) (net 25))
 (segment (start 165.1 35.56) (end 165.1 67.31) (width 0.508) (layer F.Cu) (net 25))
 (segment (start 165.1 67.31) (end 158.75 67.31) (width 0.508) (layer F.Cu) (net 25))
 (segment (start 134.79018 67.48018) (end 134.79018 70.1675) (width 0.508) (layer F.Cu) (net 25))
 (segment (start 134.62 67.31) (end 134.79018 67.48018) (width 0.508) (layer F.Cu) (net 25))
 (segment (start 158.75 67.31) (end 134.62 67.31) (width 0.508) (layer F.Cu) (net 25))
 (segment (start 78.74 69.469) (end 78.74 65.024) (width 0.508) (layer F.Cu) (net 26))
 (segment (start 101.6 40.64) (end 67.31 40.64) (width 0.508) (layer F.Cu) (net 27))
 (segment (start 67.31 40.64) (end 52.235 55.715) (width 0.508) (layer F.Cu) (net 27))
 (segment (start 52.235 55.715) (end 51.78 55.715) (width 0.508) (layer F.Cu) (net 27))
 (segment (start 101.6 40.64) (end 101.6 54.356) (width 0.508) (layer F.Cu) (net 27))
 (segment (start 101.435 40.475) (end 101.6 40.64) (width 0.508) (layer F.Cu) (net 27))
 (segment (start 106.68 44.831) (end 106.68 54.356) (width 0.381) (layer F.Cu) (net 32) (status C00000))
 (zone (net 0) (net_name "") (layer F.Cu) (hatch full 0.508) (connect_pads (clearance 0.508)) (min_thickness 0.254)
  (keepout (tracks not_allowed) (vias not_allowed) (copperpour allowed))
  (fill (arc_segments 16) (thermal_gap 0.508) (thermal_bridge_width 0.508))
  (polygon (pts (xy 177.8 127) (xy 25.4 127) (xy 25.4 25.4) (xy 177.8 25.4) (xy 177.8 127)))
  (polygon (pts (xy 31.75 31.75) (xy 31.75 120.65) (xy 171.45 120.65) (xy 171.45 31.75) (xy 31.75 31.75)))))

